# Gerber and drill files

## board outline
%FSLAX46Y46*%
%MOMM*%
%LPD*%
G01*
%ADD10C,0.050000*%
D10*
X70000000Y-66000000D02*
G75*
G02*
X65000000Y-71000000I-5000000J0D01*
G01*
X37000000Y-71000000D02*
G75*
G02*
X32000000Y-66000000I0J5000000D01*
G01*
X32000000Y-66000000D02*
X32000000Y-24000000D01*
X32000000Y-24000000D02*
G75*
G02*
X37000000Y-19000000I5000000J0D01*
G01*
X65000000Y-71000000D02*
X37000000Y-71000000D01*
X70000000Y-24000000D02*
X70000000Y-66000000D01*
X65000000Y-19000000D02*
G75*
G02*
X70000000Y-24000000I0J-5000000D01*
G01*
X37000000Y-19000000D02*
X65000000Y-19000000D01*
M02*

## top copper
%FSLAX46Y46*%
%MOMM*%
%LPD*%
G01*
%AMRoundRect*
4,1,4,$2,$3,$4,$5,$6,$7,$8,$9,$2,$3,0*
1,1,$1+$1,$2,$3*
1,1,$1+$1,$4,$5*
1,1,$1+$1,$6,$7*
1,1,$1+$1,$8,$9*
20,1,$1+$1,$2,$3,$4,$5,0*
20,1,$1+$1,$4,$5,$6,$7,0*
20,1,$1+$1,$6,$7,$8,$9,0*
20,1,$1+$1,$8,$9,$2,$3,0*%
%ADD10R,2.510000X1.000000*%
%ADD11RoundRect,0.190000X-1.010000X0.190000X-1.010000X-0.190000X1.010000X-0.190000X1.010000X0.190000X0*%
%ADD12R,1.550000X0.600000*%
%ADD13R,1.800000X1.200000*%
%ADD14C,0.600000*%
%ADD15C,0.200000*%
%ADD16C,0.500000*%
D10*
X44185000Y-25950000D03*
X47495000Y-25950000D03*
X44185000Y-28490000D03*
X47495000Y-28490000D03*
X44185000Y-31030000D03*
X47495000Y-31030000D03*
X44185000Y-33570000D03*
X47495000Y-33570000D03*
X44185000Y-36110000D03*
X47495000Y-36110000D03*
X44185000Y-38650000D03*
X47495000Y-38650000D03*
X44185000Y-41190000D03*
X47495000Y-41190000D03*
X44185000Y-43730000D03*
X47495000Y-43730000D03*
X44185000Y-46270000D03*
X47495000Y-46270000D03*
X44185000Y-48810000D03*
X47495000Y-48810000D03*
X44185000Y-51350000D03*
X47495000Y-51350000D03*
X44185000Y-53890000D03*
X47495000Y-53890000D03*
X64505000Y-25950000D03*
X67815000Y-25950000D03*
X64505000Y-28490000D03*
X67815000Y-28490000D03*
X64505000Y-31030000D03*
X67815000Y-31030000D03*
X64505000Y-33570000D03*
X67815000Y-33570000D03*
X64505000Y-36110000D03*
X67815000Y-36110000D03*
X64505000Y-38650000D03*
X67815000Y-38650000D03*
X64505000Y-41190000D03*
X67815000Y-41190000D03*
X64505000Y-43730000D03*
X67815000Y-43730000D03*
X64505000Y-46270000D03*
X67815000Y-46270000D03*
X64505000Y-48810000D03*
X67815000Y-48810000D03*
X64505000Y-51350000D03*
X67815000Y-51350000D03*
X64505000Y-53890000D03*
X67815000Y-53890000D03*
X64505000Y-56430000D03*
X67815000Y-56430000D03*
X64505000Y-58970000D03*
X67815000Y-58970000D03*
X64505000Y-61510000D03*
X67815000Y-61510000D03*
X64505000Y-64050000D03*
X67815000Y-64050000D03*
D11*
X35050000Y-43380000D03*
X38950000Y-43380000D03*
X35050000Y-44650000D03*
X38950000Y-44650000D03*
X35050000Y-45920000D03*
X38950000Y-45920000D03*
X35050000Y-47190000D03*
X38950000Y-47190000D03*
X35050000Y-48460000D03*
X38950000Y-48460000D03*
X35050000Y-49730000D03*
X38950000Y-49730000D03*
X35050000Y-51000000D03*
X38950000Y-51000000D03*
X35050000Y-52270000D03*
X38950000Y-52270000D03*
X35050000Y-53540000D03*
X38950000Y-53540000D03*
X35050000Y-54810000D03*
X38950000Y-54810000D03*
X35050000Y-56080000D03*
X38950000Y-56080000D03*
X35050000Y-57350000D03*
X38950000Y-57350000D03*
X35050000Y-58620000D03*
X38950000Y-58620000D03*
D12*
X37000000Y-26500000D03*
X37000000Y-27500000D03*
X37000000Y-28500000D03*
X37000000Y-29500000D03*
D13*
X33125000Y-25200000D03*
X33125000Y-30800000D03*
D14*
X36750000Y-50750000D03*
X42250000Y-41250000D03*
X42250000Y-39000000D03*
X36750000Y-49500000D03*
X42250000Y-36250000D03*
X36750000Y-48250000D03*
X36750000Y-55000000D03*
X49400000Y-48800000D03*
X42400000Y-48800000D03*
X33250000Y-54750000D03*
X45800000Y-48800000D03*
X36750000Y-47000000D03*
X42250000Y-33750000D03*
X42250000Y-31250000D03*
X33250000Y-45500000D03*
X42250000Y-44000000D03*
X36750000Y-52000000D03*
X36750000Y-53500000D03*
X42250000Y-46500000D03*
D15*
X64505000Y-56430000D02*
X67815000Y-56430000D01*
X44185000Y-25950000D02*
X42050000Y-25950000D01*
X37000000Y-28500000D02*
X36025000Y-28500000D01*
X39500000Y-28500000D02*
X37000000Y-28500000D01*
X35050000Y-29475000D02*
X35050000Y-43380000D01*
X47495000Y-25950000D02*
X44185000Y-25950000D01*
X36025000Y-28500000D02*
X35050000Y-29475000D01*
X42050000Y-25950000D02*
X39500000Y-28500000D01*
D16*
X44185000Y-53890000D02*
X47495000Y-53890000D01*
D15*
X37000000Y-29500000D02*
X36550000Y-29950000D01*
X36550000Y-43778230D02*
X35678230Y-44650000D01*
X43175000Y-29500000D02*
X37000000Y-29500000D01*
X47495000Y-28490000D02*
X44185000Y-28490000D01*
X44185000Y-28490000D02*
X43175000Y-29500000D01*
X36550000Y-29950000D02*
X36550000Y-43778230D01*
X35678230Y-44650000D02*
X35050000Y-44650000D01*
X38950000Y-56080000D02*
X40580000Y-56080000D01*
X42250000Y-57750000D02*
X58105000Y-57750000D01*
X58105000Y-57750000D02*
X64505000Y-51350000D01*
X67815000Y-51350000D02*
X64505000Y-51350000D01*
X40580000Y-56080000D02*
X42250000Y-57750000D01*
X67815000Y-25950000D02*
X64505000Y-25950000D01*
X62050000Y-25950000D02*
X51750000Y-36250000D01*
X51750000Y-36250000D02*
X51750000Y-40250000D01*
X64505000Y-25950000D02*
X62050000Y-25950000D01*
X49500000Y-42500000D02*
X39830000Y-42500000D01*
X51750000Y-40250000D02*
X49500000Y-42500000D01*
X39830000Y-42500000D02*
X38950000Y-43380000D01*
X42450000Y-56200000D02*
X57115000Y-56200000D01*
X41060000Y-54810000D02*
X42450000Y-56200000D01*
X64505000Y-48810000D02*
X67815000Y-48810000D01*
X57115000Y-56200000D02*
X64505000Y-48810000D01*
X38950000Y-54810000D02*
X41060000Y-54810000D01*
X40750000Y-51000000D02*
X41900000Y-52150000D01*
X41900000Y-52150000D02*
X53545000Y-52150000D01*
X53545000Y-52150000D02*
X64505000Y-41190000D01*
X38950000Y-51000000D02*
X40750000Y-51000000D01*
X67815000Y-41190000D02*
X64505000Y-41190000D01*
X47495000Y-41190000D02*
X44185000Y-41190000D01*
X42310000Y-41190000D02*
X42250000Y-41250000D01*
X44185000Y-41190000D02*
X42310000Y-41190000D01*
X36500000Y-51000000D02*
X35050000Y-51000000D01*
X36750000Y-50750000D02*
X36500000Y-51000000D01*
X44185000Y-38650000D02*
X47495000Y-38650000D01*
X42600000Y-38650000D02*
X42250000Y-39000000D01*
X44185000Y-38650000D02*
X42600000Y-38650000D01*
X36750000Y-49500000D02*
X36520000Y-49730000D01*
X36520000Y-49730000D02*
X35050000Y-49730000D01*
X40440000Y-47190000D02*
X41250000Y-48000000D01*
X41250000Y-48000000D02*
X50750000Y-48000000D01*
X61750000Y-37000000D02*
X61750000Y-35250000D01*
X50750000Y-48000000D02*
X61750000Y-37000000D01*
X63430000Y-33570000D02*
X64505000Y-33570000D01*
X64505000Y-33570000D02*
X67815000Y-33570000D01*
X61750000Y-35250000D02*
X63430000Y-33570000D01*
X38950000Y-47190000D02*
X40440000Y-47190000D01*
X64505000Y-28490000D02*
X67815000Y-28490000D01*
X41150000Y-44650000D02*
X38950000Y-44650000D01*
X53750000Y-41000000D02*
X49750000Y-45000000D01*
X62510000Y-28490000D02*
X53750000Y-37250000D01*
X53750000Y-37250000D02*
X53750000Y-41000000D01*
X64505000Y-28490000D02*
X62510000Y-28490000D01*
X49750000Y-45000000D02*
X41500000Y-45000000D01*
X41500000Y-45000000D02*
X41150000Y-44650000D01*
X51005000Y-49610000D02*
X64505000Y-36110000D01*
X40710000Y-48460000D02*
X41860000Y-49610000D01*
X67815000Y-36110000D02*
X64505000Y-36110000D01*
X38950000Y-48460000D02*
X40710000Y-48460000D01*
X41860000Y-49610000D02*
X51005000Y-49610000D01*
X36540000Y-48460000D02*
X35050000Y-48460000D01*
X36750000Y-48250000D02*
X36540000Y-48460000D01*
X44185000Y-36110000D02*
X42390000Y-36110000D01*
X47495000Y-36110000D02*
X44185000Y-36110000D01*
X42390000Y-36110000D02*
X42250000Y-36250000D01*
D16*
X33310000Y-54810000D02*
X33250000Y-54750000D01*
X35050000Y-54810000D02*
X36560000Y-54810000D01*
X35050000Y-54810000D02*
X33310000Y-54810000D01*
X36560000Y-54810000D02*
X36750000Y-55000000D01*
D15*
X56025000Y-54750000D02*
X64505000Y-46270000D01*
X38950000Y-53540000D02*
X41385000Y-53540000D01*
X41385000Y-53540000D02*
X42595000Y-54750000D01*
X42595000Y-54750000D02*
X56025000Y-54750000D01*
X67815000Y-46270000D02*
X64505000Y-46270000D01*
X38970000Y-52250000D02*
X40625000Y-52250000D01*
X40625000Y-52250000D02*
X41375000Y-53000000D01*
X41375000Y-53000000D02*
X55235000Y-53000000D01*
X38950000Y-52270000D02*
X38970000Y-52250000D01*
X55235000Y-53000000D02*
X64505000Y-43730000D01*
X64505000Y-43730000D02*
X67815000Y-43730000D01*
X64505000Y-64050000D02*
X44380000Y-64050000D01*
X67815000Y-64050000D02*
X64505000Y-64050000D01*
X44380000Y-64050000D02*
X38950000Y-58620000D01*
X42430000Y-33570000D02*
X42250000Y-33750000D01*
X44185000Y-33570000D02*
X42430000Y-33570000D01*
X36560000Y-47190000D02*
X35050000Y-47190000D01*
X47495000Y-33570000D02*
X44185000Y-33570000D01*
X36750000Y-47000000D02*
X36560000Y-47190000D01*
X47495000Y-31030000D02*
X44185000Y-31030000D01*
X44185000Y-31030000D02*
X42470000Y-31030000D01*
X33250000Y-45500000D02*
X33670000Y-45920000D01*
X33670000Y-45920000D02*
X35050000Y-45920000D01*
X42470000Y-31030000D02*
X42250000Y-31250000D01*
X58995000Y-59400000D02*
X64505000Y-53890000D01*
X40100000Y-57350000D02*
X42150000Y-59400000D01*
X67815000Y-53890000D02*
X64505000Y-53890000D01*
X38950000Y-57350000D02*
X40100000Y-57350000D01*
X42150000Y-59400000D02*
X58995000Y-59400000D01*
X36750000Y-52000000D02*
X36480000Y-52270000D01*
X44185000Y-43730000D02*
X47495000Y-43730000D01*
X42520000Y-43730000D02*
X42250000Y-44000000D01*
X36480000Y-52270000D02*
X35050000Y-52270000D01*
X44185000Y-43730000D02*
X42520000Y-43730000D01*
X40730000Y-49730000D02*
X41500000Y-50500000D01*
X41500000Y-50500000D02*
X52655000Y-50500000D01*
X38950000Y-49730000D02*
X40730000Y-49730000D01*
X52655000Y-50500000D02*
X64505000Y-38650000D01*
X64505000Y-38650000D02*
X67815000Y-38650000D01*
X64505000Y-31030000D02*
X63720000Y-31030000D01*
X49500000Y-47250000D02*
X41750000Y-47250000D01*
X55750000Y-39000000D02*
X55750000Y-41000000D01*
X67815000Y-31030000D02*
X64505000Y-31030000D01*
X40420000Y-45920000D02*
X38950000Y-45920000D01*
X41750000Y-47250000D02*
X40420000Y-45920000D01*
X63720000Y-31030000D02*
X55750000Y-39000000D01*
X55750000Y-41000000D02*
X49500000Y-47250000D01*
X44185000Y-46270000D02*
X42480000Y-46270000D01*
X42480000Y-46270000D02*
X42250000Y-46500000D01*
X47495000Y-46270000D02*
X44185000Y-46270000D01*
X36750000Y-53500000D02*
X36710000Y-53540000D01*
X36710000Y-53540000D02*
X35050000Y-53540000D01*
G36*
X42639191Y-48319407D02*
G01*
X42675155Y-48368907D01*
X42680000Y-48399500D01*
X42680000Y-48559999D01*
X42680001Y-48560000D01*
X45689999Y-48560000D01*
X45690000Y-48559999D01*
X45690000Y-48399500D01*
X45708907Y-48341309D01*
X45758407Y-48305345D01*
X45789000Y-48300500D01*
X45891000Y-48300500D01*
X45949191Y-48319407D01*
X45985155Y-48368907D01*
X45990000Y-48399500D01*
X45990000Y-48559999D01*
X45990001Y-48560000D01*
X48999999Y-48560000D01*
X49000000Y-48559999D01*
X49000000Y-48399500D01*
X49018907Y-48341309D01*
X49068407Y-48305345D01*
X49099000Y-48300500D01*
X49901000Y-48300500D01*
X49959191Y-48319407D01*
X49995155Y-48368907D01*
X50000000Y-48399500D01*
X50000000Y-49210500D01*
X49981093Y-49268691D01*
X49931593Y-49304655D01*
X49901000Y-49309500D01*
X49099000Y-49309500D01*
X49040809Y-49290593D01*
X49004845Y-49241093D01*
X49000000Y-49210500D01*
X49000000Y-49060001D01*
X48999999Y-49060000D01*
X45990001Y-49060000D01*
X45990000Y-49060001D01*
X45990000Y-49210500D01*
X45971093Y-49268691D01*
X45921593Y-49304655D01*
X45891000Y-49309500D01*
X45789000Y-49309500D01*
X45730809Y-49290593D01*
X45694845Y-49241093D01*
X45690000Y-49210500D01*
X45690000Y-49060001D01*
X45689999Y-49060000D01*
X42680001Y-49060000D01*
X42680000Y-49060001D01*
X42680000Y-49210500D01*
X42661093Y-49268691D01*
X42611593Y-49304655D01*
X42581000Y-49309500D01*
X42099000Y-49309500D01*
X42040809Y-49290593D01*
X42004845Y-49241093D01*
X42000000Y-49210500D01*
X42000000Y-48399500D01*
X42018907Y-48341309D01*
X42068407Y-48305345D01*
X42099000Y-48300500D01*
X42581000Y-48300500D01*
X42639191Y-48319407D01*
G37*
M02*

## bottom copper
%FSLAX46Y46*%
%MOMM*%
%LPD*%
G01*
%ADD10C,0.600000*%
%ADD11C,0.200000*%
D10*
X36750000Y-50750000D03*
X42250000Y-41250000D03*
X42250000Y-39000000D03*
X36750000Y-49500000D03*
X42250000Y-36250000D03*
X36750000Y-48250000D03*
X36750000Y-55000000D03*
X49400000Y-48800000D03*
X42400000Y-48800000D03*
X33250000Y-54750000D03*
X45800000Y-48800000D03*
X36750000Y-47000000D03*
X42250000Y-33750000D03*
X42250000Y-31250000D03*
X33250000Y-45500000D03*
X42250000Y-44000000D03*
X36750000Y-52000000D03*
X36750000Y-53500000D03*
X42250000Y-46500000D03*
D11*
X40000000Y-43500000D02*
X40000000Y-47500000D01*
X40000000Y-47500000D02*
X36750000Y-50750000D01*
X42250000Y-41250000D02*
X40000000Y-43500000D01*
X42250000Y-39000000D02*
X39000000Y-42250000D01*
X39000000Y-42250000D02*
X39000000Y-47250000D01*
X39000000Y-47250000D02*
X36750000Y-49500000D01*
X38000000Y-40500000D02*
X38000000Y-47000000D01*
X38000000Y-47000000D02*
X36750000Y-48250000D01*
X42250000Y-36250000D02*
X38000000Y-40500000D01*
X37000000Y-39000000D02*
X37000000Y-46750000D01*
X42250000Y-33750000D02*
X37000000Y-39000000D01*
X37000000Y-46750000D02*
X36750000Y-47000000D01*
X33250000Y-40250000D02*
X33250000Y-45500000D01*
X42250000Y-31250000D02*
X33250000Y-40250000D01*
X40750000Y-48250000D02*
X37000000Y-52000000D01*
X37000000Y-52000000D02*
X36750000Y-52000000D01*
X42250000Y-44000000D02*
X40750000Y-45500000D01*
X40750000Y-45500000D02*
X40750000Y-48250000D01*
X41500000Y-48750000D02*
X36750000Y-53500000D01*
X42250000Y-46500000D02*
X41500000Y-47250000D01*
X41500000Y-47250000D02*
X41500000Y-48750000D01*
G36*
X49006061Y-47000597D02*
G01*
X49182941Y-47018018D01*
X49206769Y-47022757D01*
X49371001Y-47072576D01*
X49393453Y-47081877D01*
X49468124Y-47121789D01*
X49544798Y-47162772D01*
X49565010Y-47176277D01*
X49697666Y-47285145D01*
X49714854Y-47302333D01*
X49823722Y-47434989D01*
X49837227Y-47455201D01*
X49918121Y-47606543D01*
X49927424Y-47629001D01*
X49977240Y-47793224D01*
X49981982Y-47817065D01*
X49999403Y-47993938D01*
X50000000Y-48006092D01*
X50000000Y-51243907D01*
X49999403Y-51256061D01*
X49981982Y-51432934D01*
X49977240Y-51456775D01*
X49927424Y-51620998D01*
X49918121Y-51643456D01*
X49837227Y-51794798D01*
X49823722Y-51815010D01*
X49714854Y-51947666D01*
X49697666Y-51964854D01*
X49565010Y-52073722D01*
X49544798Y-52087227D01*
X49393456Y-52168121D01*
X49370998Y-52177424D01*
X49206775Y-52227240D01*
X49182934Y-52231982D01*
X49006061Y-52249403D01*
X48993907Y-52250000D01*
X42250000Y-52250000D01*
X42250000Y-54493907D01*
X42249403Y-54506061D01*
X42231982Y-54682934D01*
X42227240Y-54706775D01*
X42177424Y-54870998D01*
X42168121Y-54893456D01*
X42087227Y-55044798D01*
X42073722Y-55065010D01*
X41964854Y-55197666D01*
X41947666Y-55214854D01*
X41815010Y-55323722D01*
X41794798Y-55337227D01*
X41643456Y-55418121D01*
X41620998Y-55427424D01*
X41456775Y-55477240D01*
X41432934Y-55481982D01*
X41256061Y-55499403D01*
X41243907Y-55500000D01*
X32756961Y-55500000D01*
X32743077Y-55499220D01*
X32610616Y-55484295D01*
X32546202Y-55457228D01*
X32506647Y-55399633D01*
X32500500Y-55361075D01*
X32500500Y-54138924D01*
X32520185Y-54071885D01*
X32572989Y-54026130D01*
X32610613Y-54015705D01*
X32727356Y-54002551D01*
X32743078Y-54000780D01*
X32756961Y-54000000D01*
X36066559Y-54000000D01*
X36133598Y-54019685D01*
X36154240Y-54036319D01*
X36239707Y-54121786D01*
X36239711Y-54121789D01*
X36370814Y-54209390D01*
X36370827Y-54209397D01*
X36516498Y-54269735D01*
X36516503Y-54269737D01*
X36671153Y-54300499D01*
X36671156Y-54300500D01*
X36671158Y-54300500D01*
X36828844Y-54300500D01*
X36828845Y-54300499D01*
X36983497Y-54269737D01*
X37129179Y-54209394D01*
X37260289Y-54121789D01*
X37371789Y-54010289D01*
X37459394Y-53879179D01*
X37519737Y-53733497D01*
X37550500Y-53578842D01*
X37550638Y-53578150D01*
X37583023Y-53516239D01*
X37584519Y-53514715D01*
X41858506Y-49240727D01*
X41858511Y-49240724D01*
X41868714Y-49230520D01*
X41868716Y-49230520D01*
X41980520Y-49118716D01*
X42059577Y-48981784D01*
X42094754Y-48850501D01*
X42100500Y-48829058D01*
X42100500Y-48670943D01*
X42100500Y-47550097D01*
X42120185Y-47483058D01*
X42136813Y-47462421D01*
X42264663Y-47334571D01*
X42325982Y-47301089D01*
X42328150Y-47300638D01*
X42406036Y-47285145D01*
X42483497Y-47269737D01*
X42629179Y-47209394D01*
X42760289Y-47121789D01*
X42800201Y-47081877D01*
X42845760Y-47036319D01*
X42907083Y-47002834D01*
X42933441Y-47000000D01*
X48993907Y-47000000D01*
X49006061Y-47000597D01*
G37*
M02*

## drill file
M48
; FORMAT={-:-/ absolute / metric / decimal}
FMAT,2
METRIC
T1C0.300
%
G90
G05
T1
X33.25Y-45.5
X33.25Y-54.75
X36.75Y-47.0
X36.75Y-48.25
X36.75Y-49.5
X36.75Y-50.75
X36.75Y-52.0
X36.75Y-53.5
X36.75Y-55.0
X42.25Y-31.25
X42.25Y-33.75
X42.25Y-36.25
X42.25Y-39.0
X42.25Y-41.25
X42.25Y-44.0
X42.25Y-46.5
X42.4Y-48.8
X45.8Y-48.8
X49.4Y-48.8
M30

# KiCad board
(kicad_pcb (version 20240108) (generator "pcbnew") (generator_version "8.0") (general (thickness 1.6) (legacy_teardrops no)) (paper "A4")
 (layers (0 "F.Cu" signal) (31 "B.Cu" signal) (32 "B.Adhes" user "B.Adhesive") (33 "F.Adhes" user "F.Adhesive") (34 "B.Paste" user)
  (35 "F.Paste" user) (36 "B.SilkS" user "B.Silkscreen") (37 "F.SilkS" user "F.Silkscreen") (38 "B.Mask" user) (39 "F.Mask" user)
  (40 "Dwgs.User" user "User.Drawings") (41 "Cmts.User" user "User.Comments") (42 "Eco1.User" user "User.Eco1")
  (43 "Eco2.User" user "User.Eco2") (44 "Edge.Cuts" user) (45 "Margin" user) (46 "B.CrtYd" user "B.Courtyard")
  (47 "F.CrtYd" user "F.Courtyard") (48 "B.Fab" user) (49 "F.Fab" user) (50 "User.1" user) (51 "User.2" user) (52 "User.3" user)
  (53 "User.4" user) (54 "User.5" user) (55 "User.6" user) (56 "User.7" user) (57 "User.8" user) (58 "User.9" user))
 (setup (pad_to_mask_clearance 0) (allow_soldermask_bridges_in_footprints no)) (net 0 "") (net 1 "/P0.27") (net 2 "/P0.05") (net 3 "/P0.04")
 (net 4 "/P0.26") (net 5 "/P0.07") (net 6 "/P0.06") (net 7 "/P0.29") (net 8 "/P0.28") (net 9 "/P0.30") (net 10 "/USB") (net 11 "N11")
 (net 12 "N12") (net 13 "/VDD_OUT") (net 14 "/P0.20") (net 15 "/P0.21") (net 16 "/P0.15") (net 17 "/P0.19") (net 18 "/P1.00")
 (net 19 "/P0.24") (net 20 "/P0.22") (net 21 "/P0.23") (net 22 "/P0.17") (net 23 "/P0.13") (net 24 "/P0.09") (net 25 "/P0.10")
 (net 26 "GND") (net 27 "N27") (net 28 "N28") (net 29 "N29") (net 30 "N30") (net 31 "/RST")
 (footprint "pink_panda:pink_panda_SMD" (layer "F.Cu") (at 56 45)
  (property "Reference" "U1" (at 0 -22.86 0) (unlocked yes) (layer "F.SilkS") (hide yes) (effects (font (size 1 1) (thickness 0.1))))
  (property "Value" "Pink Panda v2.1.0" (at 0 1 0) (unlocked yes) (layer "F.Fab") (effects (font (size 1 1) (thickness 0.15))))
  (pad "1" smd rect (at -11.815 -19.05) (size 2.51 1) (layers "F.Cu" "F.Paste" "F.Mask") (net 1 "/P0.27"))
  (pad "1" smd rect (at -8.505 -19.05) (size 2.51 1) (layers "F.Cu" "F.Paste" "F.Mask") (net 1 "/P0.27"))
  (pad "2" smd rect (at -11.815 -16.51) (size 2.51 1) (layers "F.Cu" "F.Paste" "F.Mask") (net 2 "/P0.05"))
  (pad "2" smd rect (at -8.505 -16.51) (size 2.51 1) (layers "F.Cu" "F.Paste" "F.Mask") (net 2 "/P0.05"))
  (pad "3" smd rect (at -11.815 -13.97) (size 2.51 1) (layers "F.Cu" "F.Paste" "F.Mask") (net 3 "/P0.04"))
  (pad "3" smd rect (at -8.505 -13.97) (size 2.51 1) (layers "F.Cu" "F.Paste" "F.Mask") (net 3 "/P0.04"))
  (pad "4" smd rect (at -11.815 -11.43) (size 2.51 1) (layers "F.Cu" "F.Paste" "F.Mask") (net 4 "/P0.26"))
  (pad "4" smd rect (at -8.505 -11.43) (size 2.51 1) (layers "F.Cu" "F.Paste" "F.Mask") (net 4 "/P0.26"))
  (pad "5" smd rect (at -11.815 -8.89) (size 2.51 1) (layers "F.Cu" "F.Paste" "F.Mask") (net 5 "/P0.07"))
  (pad "5" smd rect (at -8.505 -8.89) (size 2.51 1) (layers "F.Cu" "F.Paste" "F.Mask") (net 5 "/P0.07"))
  (pad "6" smd rect (at -11.815 -6.35) (size 2.51 1) (layers "F.Cu" "F.Paste" "F.Mask") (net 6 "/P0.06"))
  (pad "6" smd rect (at -8.505 -6.35) (size 2.51 1) (layers "F.Cu" "F.Paste" "F.Mask") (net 6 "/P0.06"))
  (pad "7" smd rect (at -11.815 -3.81) (size 2.51 1) (layers "F.Cu" "F.Paste" "F.Mask") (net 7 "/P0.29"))
  (pad "7" smd rect (at -8.505 -3.81) (size 2.51 1) (layers "F.Cu" "F.Paste" "F.Mask") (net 7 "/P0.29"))
  (pad "8" smd rect (at -11.815 -1.27) (size 2.51 1) (layers "F.Cu" "F.Paste" "F.Mask") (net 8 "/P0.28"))
  (pad "8" smd rect (at -8.505 -1.27) (size 2.51 1) (layers "F.Cu" "F.Paste" "F.Mask") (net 8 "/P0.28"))
  (pad "9" smd rect (at -11.815 1.27) (size 2.51 1) (layers "F.Cu" "F.Paste" "F.Mask") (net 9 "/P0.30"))
  (pad "9" smd rect (at -8.505 1.27) (size 2.51 1) (layers "F.Cu" "F.Paste" "F.Mask") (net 9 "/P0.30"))
  (pad "10" smd rect (at -11.815 3.81) (size 2.51 1) (layers "F.Cu" "F.Paste" "F.Mask") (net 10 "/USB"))
  (pad "10" smd rect (at -8.505 3.81) (size 2.51 1) (layers "F.Cu" "F.Paste" "F.Mask") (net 10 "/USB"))
  (pad "11" smd rect (at -11.815 6.35) (size 2.51 1) (layers "F.Cu" "F.Paste" "F.Mask") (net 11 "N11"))
  (pad "11" smd rect (at -8.505 6.35) (size 2.51 1) (layers "F.Cu" "F.Paste" "F.Mask") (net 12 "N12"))
  (pad "12" smd rect (at -11.815 8.89) (size 2.51 1) (layers "F.Cu" "F.Paste" "F.Mask") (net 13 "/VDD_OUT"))
  (pad "12" smd rect (at -8.505 8.89) (size 2.51 1) (layers "F.Cu" "F.Paste" "F.Mask") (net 13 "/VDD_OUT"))
  (pad "13" smd rect (at 8.505 -19.05) (size 2.51 1) (layers "F.Cu" "F.Paste" "F.Mask") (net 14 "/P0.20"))
  (pad "13" smd rect (at 11.815 -19.05) (size 2.51 1) (layers "F.Cu" "F.Paste" "F.Mask") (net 14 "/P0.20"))
  (pad "14" smd rect (at 8.505 -16.51) (size 2.51 1) (layers "F.Cu" "F.Paste" "F.Mask") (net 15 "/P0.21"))
  (pad "14" smd rect (at 11.815 -16.51) (size 2.51 1) (layers "F.Cu" "F.Paste" "F.Mask") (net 15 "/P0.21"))
  (pad "15" smd rect (at 8.505 -13.97) (size 2.51 1) (layers "F.Cu" "F.Paste" "F.Mask") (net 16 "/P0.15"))
  (pad "15" smd rect (at 11.815 -13.97) (size 2.51 1) (layers "F.Cu" "F.Paste" "F.Mask") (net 16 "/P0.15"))
  (pad "16" smd rect (at 8.505 -11.43) (size 2.51 1) (layers "F.Cu" "F.Paste" "F.Mask") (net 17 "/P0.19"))
  (pad "16" smd rect (at 11.815 -11.43) (size 2.51 1) (layers "F.Cu" "F.Paste" "F.Mask") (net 17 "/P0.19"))
  (pad "17" smd rect (at 8.505 -8.89) (size 2.51 1) (layers "F.Cu" "F.Paste" "F.Mask") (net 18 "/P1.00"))
  (pad "17" smd rect (at 11.815 -8.89) (size 2.51 1) (layers "F.Cu" "F.Paste" "F.Mask") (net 18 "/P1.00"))
  (pad "18" smd rect (at 8.505 -6.35) (size 2.51 1) (layers "F.Cu" "F.Paste" "F.Mask") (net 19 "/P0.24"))
  (pad "18" smd rect (at 11.815 -6.35) (size 2.51 1) (layers "F.Cu" "F.Paste" "F.Mask") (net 19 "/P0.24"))
  (pad "19" smd rect (at 8.505 -3.81) (size 2.51 1) (layers "F.Cu" "F.Paste" "F.Mask") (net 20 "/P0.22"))
  (pad "19" smd rect (at 11.815 -3.81) (size 2.51 1) (layers "F.Cu" "F.Paste" "F.Mask") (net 20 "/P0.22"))
  (pad "20" smd rect (at 8.505 -1.27) (size 2.51 1) (layers "F.Cu" "F.Paste" "F.Mask") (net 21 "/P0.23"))
  (pad "20" smd rect (at 11.815 -1.27) (size 2.51 1) (layers "F.Cu" "F.Paste" "F.Mask") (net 21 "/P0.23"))
  (pad "21" smd rect (at 8.505 1.27) (size 2.51 1) (layers "F.Cu" "F.Paste" "F.Mask") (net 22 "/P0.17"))
  (pad "21" smd rect (at 11.815 1.27) (size 2.51 1) (layers "F.Cu" "F.Paste" "F.Mask") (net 22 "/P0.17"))
  (pad "22" smd rect (at 8.505 3.81) (size 2.51 1) (layers "F.Cu" "F.Paste" "F.Mask") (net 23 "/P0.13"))
  (pad "22" smd rect (at 11.815 3.81) (size 2.51 1) (layers "F.Cu" "F.Paste" "F.Mask") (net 23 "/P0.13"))
  (pad "23" smd rect (at 8.505 6.35) (size 2.51 1) (layers "F.Cu" "F.Paste" "F.Mask") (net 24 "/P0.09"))
  (pad "23" smd rect (at 11.815 6.35) (size 2.51 1) (layers "F.Cu" "F.Paste" "F.Mask") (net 24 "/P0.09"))
  (pad "24" smd rect (at 8.505 8.89) (size 2.51 1) (layers "F.Cu" "F.Paste" "F.Mask") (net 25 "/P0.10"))
  (pad "24" smd rect (at 11.815 8.89) (size 2.51 1) (layers "F.Cu" "F.Paste" "F.Mask") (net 25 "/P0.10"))
  (pad "25" smd rect (at 8.505 11.43) (size 2.51 1) (layers "F.Cu" "F.Paste" "F.Mask") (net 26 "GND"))
  (pad "25" smd rect (at 11.815 11.43) (size 2.51 1) (layers "F.Cu" "F.Paste" "F.Mask") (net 26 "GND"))
  (pad "26" smd rect (at 8.505 13.97) (size 2.51 1) (layers "F.Cu" "F.Paste" "F.Mask") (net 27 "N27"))
  (pad "26" smd rect (at 11.815 13.97) (size 2.51 1) (layers "F.Cu" "F.Paste" "F.Mask") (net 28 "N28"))
  (pad "27" smd rect (at 8.505 16.51) (size 2.51 1) (layers "F.Cu" "F.Paste" "F.Mask") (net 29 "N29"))
  (pad "27" smd rect (at 11.815 16.51) (size 2.51 1) (layers "F.Cu" "F.Paste" "F.Mask") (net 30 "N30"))
  (pad "28" smd rect (at 8.505 19.05) (size 2.51 1) (layers "F.Cu" "F.Paste" "F.Mask") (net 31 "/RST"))
  (pad "28" smd rect (at 11.815 19.05) (size 2.51 1) (layers "F.Cu" "F.Paste" "F.Mask") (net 31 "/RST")))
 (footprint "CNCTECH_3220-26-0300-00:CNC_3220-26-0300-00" (layer "F.Cu") (at 37 51 -90)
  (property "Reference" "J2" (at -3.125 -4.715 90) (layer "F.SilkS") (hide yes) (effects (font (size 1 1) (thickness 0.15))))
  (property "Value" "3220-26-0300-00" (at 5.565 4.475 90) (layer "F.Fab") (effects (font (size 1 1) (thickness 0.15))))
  (pad "1" smd roundrect (at -7.62 1.95 270) (size 0.76 2.4) (layers "F.Cu" "F.Paste" "F.Mask") (roundrect_rratio 0.25) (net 1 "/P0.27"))
  (pad "2" smd roundrect (at -7.62 -1.95 270) (size 0.76 2.4) (layers "F.Cu" "F.Paste" "F.Mask") (roundrect_rratio 0.25) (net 14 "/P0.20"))
  (pad "3" smd roundrect (at -6.35 1.95 270) (size 0.76 2.4) (layers "F.Cu" "F.Paste" "F.Mask") (roundrect_rratio 0.25) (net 2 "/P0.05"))
  (pad "4" smd roundrect (at -6.35 -1.95 270) (size 0.76 2.4) (layers "F.Cu" "F.Paste" "F.Mask") (roundrect_rratio 0.25) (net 15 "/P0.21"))
  (pad "5" smd roundrect (at -5.08 1.95 270) (size 0.76 2.4) (layers "F.Cu" "F.Paste" "F.Mask") (roundrect_rratio 0.25) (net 3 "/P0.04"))
  (pad "6" smd roundrect (at -5.08 -1.95 270) (size 0.76 2.4) (layers "F.Cu" "F.Paste" "F.Mask") (roundrect_rratio 0.25) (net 16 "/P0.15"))
  (pad "7" smd roundrect (at -3.81 1.95 270) (size 0.76 2.4) (layers "F.Cu" "F.Paste" "F.Mask") (roundrect_rratio 0.25) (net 4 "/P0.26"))
  (pad "8" smd roundrect (at -3.81 -1.95 270) (size 0.76 2.4) (layers "F.Cu" "F.Paste" "F.Mask") (roundrect_rratio 0.25) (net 17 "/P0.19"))
  (pad "9" smd roundrect (at -2.54 1.95 270) (size 0.76 2.4) (layers "F.Cu" "F.Paste" "F.Mask") (roundrect_rratio 0.25) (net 5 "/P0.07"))
  (pad "10" smd roundrect (at -2.54 -1.95 270) (size 0.76 2.4) (layers "F.Cu" "F.Paste" "F.Mask") (roundrect_rratio 0.25) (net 18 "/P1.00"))
  (pad "11" smd roundrect (at -1.27 1.95 270) (size 0.76 2.4) (layers "F.Cu" "F.Paste" "F.Mask") (roundrect_rratio 0.25) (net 6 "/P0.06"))
  (pad "12" smd roundrect (at -1.27 -1.95 270) (size 0.76 2.4) (layers "F.Cu" "F.Paste" "F.Mask") (roundrect_rratio 0.25) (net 19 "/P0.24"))
  (pad "13" smd roundrect (at 0 1.95 270) (size 0.76 2.4) (layers "F.Cu" "F.Paste" "F.Mask") (roundrect_rratio 0.25) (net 7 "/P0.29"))
  (pad "14" smd roundrect (at 0 -1.95 270) (size 0.76 2.4) (layers "F.Cu" "F.Paste" "F.Mask") (roundrect_rratio 0.25) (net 20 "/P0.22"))
  (pad "15" smd roundrect (at 1.27 1.95 270) (size 0.76 2.4) (layers "F.Cu" "F.Paste" "F.Mask") (roundrect_rratio 0.25) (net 8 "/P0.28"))
  (pad "16" smd roundrect (at 1.27 -1.95 270) (size 0.76 2.4) (layers "F.Cu" "F.Paste" "F.Mask") (roundrect_rratio 0.25) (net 21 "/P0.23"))
  (pad "17" smd roundrect (at 2.54 1.95 270) (size 0.76 2.4) (layers "F.Cu" "F.Paste" "F.Mask") (roundrect_rratio 0.25) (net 9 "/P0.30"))
  (pad "18" smd roundrect (at 2.54 -1.95 270) (size 0.76 2.4) (layers "F.Cu" "F.Paste" "F.Mask") (roundrect_rratio 0.25) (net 22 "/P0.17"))
  (pad "19" smd roundrect (at 3.81 1.95 270) (size 0.76 2.4) (layers "F.Cu" "F.Paste" "F.Mask") (roundrect_rratio 0.25) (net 10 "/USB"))
  (pad "20" smd roundrect (at 3.81 -1.95 270) (size 0.76 2.4) (layers "F.Cu" "F.Paste" "F.Mask") (roundrect_rratio 0.25) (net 23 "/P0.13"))
  (pad "21" smd roundrect (at 5.08 1.95 270) (size 0.76 2.4) (layers "F.Cu" "F.Paste" "F.Mask") (roundrect_rratio 0.25) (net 13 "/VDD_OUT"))
  (pad "22" smd roundrect (at 5.08 -1.95 270) (size 0.76 2.4) (layers "F.Cu" "F.Paste" "F.Mask") (roundrect_rratio 0.25) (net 24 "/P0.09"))
  (pad "23" smd roundrect (at 6.35 1.95 270) (size 0.76 2.4) (layers "F.Cu" "F.Paste" "F.Mask") (roundrect_rratio 0.25) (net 26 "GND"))
  (pad "24" smd roundrect (at 6.35 -1.95 270) (size 0.76 2.4) (layers "F.Cu" "F.Paste" "F.Mask") (roundrect_rratio 0.25) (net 25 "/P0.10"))
  (pad "25" smd roundrect (at 7.62 1.95 270) (size 0.76 2.4) (layers "F.Cu" "F.Paste" "F.Mask") (roundrect_rratio 0.25) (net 26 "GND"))
  (pad "26" smd roundrect (at 7.62 -1.95 270) (size 0.76 2.4) (layers "F.Cu" "F.Paste" "F.Mask") (roundrect_rratio 0.25) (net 31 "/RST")))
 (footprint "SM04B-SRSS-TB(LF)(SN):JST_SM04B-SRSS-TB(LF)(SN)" (layer "F.Cu") (at 37 28 -90)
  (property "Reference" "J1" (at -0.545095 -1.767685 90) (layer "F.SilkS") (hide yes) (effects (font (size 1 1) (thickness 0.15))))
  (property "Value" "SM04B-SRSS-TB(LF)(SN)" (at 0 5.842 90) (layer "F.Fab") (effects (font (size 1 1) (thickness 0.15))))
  (pad "1" smd rect (at -1.5 0 270) (size 0.6 1.55) (layers "F.Cu" "F.Paste" "F.Mask") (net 26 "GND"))
  (pad "2" smd rect (at -0.5 0 270) (size 0.6 1.55) (layers "F.Cu" "F.Paste" "F.Mask") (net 13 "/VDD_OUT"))
  (pad "3" smd rect (at 0.5 0 270) (size 0.6 1.55) (layers "F.Cu" "F.Paste" "F.Mask") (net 1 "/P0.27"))
  (pad "4" smd rect (at 1.5 0 270) (size 0.6 1.55) (layers "F.Cu" "F.Paste" "F.Mask") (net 2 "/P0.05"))
  (pad "S1" smd rect (at -2.8 3.875 270) (size 1.2 1.8) (layers "F.Cu" "F.Paste" "F.Mask") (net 26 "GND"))
  (pad "S2" smd rect (at 2.8 3.875 270) (size 1.2 1.8) (layers "F.Cu" "F.Paste" "F.Mask") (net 26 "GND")))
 (gr_arc (start 70 66) (mid 68.535534 69.535534) (end 65 71) (stroke (width 0.05) (type default)) (layer "Edge.Cuts"))
 (gr_arc (start 37 71) (mid 33.464466 69.535534) (end 32 66) (stroke (width 0.05) (type default)) (layer "Edge.Cuts"))
 (gr_line (start 32 66) (end 32 24) (stroke (width 0.05) (type default)) (layer "Edge.Cuts"))
 (gr_arc (start 32 24) (mid 33.464466 20.464466) (end 37 19) (stroke (width 0.05) (type default)) (layer "Edge.Cuts"))
 (gr_line (start 65 71) (end 37 71) (stroke (width 0.05) (type default)) (layer "Edge.Cuts"))
 (gr_line (start 70 24) (end 70 66) (stroke (width 0.05) (type default)) (layer "Edge.Cuts"))
 (gr_arc (start 65 19) (mid 68.535534 20.464466) (end 70 24) (stroke (width 0.05) (type default)) (layer "Edge.Cuts"))
 (gr_line (start 37 19) (end 65 19) (stroke (width 0.05) (type default)) (layer "Edge.Cuts"))
 (segment (start 64.505 56.43) (end 67.815 56.43) (width 0.2) (layer "F.Cu") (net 26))
 (segment (start 44.185 25.95) (end 42.05 25.95) (width 0.2) (layer "F.Cu") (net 1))
 (segment (start 37 28.5) (end 36.025 28.5) (width 0.2) (layer "F.Cu") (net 1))
 (segment (start 39.5 28.5) (end 37 28.5) (width 0.2) (layer "F.Cu") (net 1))
 (segment (start 35.05 29.475) (end 35.05 43.38) (width 0.2) (layer "F.Cu") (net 1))
 (segment (start 47.495 25.95) (end 44.185 25.95) (width 0.2) (layer "F.Cu") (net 1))
 (segment (start 36.025 28.5) (end 35.05 29.475) (width 0.2) (layer "F.Cu") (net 1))
 (segment (start 42.05 25.95) (end 39.5 28.5) (width 0.2) (layer "F.Cu") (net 1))
 (segment (start 44.185 53.89) (end 47.495 53.89) (width 0.5) (layer "F.Cu") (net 13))
 (segment (start 37 29.5) (end 36.55 29.95) (width 0.2) (layer "F.Cu") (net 2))
 (segment (start 36.55 43.77823) (end 35.67823 44.65) (width 0.2) (layer "F.Cu") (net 2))
 (segment (start 43.175 29.5) (end 37 29.5) (width 0.2) (layer "F.Cu") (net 2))
 (segment (start 47.495 28.49) (end 44.185 28.49) (width 0.2) (layer "F.Cu") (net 2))
 (segment (start 44.185 28.49) (end 43.175 29.5) (width 0.2) (layer "F.Cu") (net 2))
 (segment (start 36.55 29.95) (end 36.55 43.77823) (width 0.2) (layer "F.Cu") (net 2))
 (segment (start 35.67823 44.65) (end 35.05 44.65) (width 0.2) (layer "F.Cu") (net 2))
 (segment (start 38.95 56.08) (end 40.58 56.08) (width 0.2) (layer "F.Cu") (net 24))
 (segment (start 42.25 57.75) (end 58.105 57.75) (width 0.2) (layer "F.Cu") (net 24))
 (segment (start 58.105 57.75) (end 64.505 51.35) (width 0.2) (layer "F.Cu") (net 24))
 (segment (start 67.815 51.35) (end 64.505 51.35) (width 0.2) (layer "F.Cu") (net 24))
 (segment (start 40.58 56.08) (end 42.25 57.75) (width 0.2) (layer "F.Cu") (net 24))
 (segment (start 67.815 25.95) (end 64.505 25.95) (width 0.2) (layer "F.Cu") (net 14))
 (segment (start 62.05 25.95) (end 51.75 36.25) (width 0.2) (layer "F.Cu") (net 14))
 (segment (start 51.75 36.25) (end 51.75 40.25) (width 0.2) (layer "F.Cu") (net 14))
 (segment (start 64.505 25.95) (end 62.05 25.95) (width 0.2) (layer "F.Cu") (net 14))
 (segment (start 49.5 42.5) (end 39.83 42.5) (width 0.2) (layer "F.Cu") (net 14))
 (segment (start 51.75 40.25) (end 49.5 42.5) (width 0.2) (layer "F.Cu") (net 14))
 (segment (start 39.83 42.5) (end 38.95 43.38) (width 0.2) (layer "F.Cu") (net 14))
 (segment (start 42.45 56.2) (end 57.115 56.2) (width 0.2) (layer "F.Cu") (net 23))
 (segment (start 41.06 54.81) (end 42.45 56.2) (width 0.2) (layer "F.Cu") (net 23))
 (segment (start 64.505 48.81) (end 67.815 48.81) (width 0.2) (layer "F.Cu") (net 23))
 (segment (start 57.115 56.2) (end 64.505 48.81) (width 0.2) (layer "F.Cu") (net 23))
 (segment (start 38.95 54.81) (end 41.06 54.81) (width 0.2) (layer "F.Cu") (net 23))
 (segment (start 40.75 51) (end 41.9 52.15) (width 0.2) (layer "F.Cu") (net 20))
 (segment (start 41.9 52.15) (end 53.545 52.15) (width 0.2) (layer "F.Cu") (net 20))
 (segment (start 53.545 52.15) (end 64.505 41.19) (width 0.2) (layer "F.Cu") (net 20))
 (segment (start 38.95 51) (end 40.75 51) (width 0.2) (layer "F.Cu") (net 20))
 (segment (start 67.815 41.19) (end 64.505 41.19) (width 0.2) (layer "F.Cu") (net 20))
 (segment (start 47.495 41.19) (end 44.185 41.19) (width 0.2) (layer "F.Cu") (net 7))
 (segment (start 42.31 41.19) (end 42.25 41.25) (width 0.2) (layer "F.Cu") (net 7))
 (segment (start 44.185 41.19) (end 42.31 41.19) (width 0.2) (layer "F.Cu") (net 7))
 (segment (start 36.5 51) (end 35.05 51) (width 0.2) (layer "F.Cu") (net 7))
 (segment (start 36.75 50.75) (end 36.5 51) (width 0.2) (layer "F.Cu") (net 7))
 (via (at 36.75 50.75) (size 0.6) (drill 0.3) (layers "F.Cu" "B.Cu") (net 7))
 (via (at 42.25 41.25) (size 0.6) (drill 0.3) (layers "F.Cu" "B.Cu") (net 7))
 (segment (start 40 43.5) (end 40 47.5) (width 0.2) (layer "B.Cu") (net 7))
 (segment (start 40 47.5) (end 36.75 50.75) (width 0.2) (layer "B.Cu") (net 7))
 (segment (start 42.25 41.25) (end 40 43.5) (width 0.2) (layer "B.Cu") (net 7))
 (segment (start 44.185 38.65) (end 47.495 38.65) (width 0.2) (layer "F.Cu") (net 6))
 (segment (start 42.6 38.65) (end 42.25 39) (width 0.2) (layer "F.Cu") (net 6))
 (segment (start 44.185 38.65) (end 42.6 38.65) (width 0.2) (layer "F.Cu") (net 6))
 (segment (start 36.75 49.5) (end 36.52 49.73) (width 0.2) (layer "F.Cu") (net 6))
 (segment (start 36.52 49.73) (end 35.05 49.73) (width 0.2) (layer "F.Cu") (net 6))
 (via (at 42.25 39) (size 0.6) (drill 0.3) (layers "F.Cu" "B.Cu") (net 6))
 (via (at 36.75 49.5) (size 0.6) (drill 0.3) (layers "F.Cu" "B.Cu") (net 6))
 (segment (start 42.25 39) (end 39 42.25) (width 0.2) (layer "B.Cu") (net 6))
 (segment (start 39 42.25) (end 39 47.25) (width 0.2) (layer "B.Cu") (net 6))
 (segment (start 39 47.25) (end 36.75 49.5) (width 0.2) (layer "B.Cu") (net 6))
 (segment (start 40.44 47.19) (end 41.25 48) (width 0.2) (layer "F.Cu") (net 17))
 (segment (start 41.25 48) (end 50.75 48) (width 0.2) (layer "F.Cu") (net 17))
 (segment (start 61.75 37) (end 61.75 35.25) (width 0.2) (layer "F.Cu") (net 17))
 (segment (start 50.75 48) (end 61.75 37) (width 0.2) (layer "F.Cu") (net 17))
 (segment (start 63.43 33.57) (end 64.505 33.57) (width 0.2) (layer "F.Cu") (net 17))
 (segment (start 64.505 33.57) (end 67.815 33.57) (width 0.2) (layer "F.Cu") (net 17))
 (segment (start 61.75 35.25) (end 63.43 33.57) (width 0.2) (layer "F.Cu") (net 17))
 (segment (start 38.95 47.19) (end 40.44 47.19) (width 0.2) (layer "F.Cu") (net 17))
 (segment (start 64.505 28.49) (end 67.815 28.49) (width 0.2) (layer "F.Cu") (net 15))
 (segment (start 41.15 44.65) (end 38.95 44.65) (width 0.2) (layer "F.Cu") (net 15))
 (segment (start 53.75 41) (end 49.75 45) (width 0.2) (layer "F.Cu") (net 15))
 (segment (start 62.51 28.49) (end 53.75 37.25) (width 0.2) (layer "F.Cu") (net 15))
 (segment (start 53.75 37.25) (end 53.75 41) (width 0.2) (layer "F.Cu") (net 15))
 (segment (start 64.505 28.49) (end 62.51 28.49) (width 0.2) (layer "F.Cu") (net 15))
 (segment (start 49.75 45) (end 41.5 45) (width 0.2) (layer "F.Cu") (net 15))
 (segment (start 41.5 45) (end 41.15 44.65) (width 0.2) (layer "F.Cu") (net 15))
 (segment (start 51.005 49.61) (end 64.505 36.11) (width 0.2) (layer "F.Cu") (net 18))
 (segment (start 40.71 48.46) (end 41.86 49.61) (width 0.2) (layer "F.Cu") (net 18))
 (segment (start 67.815 36.11) (end 64.505 36.11) (width 0.2) (layer "F.Cu") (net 18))
 (segment (start 38.95 48.46) (end 40.71 48.46) (width 0.2) (layer "F.Cu") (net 18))
 (segment (start 41.86 49.61) (end 51.005 49.61) (width 0.2) (layer "F.Cu") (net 18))
 (segment (start 36.54 48.46) (end 35.05 48.46) (width 0.2) (layer "F.Cu") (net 5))
 (segment (start 36.75 48.25) (end 36.54 48.46) (width 0.2) (layer "F.Cu") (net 5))
 (segment (start 44.185 36.11) (end 42.39 36.11) (width 0.2) (layer "F.Cu") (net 5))
 (segment (start 47.495 36.11) (end 44.185 36.11) (width 0.2) (layer "F.Cu") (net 5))
 (segment (start 42.39 36.11) (end 42.25 36.25) (width 0.2) (layer "F.Cu") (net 5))
 (via (at 42.25 36.25) (size 0.6) (drill 0.3) (layers "F.Cu" "B.Cu") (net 5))
 (via (at 36.75 48.25) (size 0.6) (drill 0.3) (layers "F.Cu" "B.Cu") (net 5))
 (segment (start 38 40.5) (end 38 47) (width 0.2) (layer "B.Cu") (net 5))
 (segment (start 38 47) (end 36.75 48.25) (width 0.2) (layer "B.Cu") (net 5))
 (segment (start 42.25 36.25) (end 38 40.5) (width 0.2) (layer "B.Cu") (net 5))
 (segment (start 33.31 54.81) (end 33.25 54.75) (width 0.5) (layer "F.Cu") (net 10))
 (segment (start 35.05 54.81) (end 36.56 54.81) (width 0.5) (layer "F.Cu") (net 10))
 (segment (start 35.05 54.81) (end 33.31 54.81) (width 0.5) (layer "F.Cu") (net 10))
 (segment (start 36.56 54.81) (end 36.75 55) (width 0.5) (layer "F.Cu") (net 10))
 (via (at 36.75 55) (size 0.6) (drill 0.3) (layers "F.Cu" "B.Cu") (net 10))
 (via (at 49.4 48.8) (size 0.6) (drill 0.3) (layers "F.Cu" "B.Cu") (free yes) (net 10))
 (via (at 42.4 48.8) (size 0.6) (drill 0.3) (layers "F.Cu" "B.Cu") (free yes) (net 10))
 (via (at 33.25 54.75) (size 0.6) (drill 0.3) (layers "F.Cu" "B.Cu") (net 10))
 (via (at 45.8 48.8) (size 0.6) (drill 0.3) (layers "F.Cu" "B.Cu") (free yes) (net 10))
 (segment (start 56.025 54.75) (end 64.505 46.27) (width 0.2) (layer "F.Cu") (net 22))
 (segment (start 38.95 53.54) (end 41.385 53.54) (width 0.2) (layer "F.Cu") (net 22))
 (segment (start 41.385 53.54) (end 42.595 54.75) (width 0.2) (layer "F.Cu") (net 22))
 (segment (start 42.595 54.75) (end 56.025 54.75) (width 0.2) (layer "F.Cu") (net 22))
 (segment (start 67.815 46.27) (end 64.505 46.27) (width 0.2) (layer "F.Cu") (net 22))
 (segment (start 38.97 52.25) (end 40.625 52.25) (width 0.2) (layer "F.Cu") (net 21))
 (segment (start 40.625 52.25) (end 41.375 53) (width 0.2) (layer "F.Cu") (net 21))
 (segment (start 41.375 53) (end 55.235 53) (width 0.2) (layer "F.Cu") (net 21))
 (segment (start 38.95 52.27) (end 38.97 52.25) (width 0.2) (layer "F.Cu") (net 21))
 (segment (start 55.235 53) (end 64.505 43.73) (width 0.2) (layer "F.Cu") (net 21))
 (segment (start 64.505 43.73) (end 67.815 43.73) (width 0.2) (layer "F.Cu") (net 21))
 (segment (start 64.505 64.05) (end 44.38 64.05) (width 0.2) (layer "F.Cu") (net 31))
 (segment (start 67.815 64.05) (end 64.505 64.05) (width 0.2) (layer "F.Cu") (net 31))
 (segment (start 44.38 64.05) (end 38.95 58.62) (width 0.2) (layer "F.Cu") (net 31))
 (segment (start 42.43 33.57) (end 42.25 33.75) (width 0.2) (layer "F.Cu") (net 4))
 (segment (start 44.185 33.57) (end 42.43 33.57) (width 0.2) (layer "F.Cu") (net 4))
 (segment (start 36.56 47.19) (end 35.05 47.19) (width 0.2) (layer "F.Cu") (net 4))
 (segment (start 47.495 33.57) (end 44.185 33.57) (width 0.2) (layer "F.Cu") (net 4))
 (segment (start 36.75 47) (end 36.56 47.19) (width 0.2) (layer "F.Cu") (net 4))
 (via (at 36.75 47) (size 0.6) (drill 0.3) (layers "F.Cu" "B.Cu") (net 4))
 (via (at 42.25 33.75) (size 0.6) (drill 0.3) (layers "F.Cu" "B.Cu") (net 4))
 (segment (start 37 39) (end 37 46.75) (width 0.2) (layer "B.Cu") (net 4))
 (segment (start 42.25 33.75) (end 37 39) (width 0.2) (layer "B.Cu") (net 4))
 (segment (start 37 46.75) (end 36.75 47) (width 0.2) (layer "B.Cu") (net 4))
 (segment (start 47.495 31.03) (end 44.185 31.03) (width 0.2) (layer "F.Cu") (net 3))
 (segment (start 44.185 31.03) (end 42.47 31.03) (width 0.2) (layer "F.Cu") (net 3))
 (segment (start 33.25 45.5) (end 33.67 45.92) (width 0.2) (layer "F.Cu") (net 3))
 (segment (start 33.67 45.92) (end 35.05 45.92) (width 0.2) (layer "F.Cu") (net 3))
 (segment (start 42.47 31.03) (end 42.25 31.25) (width 0.2) (layer "F.Cu") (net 3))
 (via (at 42.25 31.25) (size 0.6) (drill 0.3) (layers "F.Cu" "B.Cu") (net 3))
 (via (at 33.25 45.5) (size 0.6) (drill 0.3) (layers "F.Cu" "B.Cu") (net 3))
 (segment (start 33.25 40.25) (end 33.25 45.5) (width 0.2) (layer "B.Cu") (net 3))
 (segment (start 42.25 31.25) (end 33.25 40.25) (width 0.2) (layer "B.Cu") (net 3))
 (segment (start 58.995 59.4) (end 64.505 53.89) (width 0.2) (layer "F.Cu") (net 25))
 (segment (start 40.1 57.35) (end 42.15 59.4) (width 0.2) (layer "F.Cu") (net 25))
 (segment (start 67.815 53.89) (end 64.505 53.89) (width 0.2) (layer "F.Cu") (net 25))
 (segment (start 38.95 57.35) (end 40.1 57.35) (width 0.2) (layer "F.Cu") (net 25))
 (segment (start 42.15 59.4) (end 58.995 59.4) (width 0.2) (layer "F.Cu") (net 25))
 (segment (start 36.75 52) (end 36.48 52.27) (width 0.2) (layer "F.Cu") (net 8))
 (segment (start 44.185 43.73) (end 47.495 43.73) (width 0.2) (layer "F.Cu") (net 8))
 (segment (start 42.52 43.73) (end 42.25 44) (width 0.2) (layer "F.Cu") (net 8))
 (segment (start 36.48 52.27) (end 35.05 52.27) (width 0.2) (layer "F.Cu") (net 8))
 (segment (start 44.185 43.73) (end 42.52 43.73) (width 0.2) (layer "F.Cu") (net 8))
 (via (at 42.25 44) (size 0.6) (drill 0.3) (layers "F.Cu" "B.Cu") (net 8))
 (via (at 36.75 52) (size 0.6) (drill 0.3) (layers "F.Cu" "B.Cu") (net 8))
 (segment (start 40.75 48.25) (end 37 52) (width 0.2) (layer "B.Cu") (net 8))
 (segment (start 37 52) (end 36.75 52) (width 0.2) (layer "B.Cu") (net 8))
 (segment (start 42.25 44) (end 40.75 45.5) (width 0.2) (layer "B.Cu") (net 8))
 (segment (start 40.75 45.5) (end 40.75 48.25) (width 0.2) (layer "B.Cu") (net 8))
 (segment (start 40.73 49.73) (end 41.5 50.5) (width 0.2) (layer "F.Cu") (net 19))
 (segment (start 41.5 50.5) (end 52.655 50.5) (width 0.2) (layer "F.Cu") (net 19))
 (segment (start 38.95 49.73) (end 40.73 49.73) (width 0.2) (layer "F.Cu") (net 19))
 (segment (start 52.655 50.5) (end 64.505 38.65) (width 0.2) (layer "F.Cu") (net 19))
 (segment (start 64.505 38.65) (end 67.815 38.65) (width 0.2) (layer "F.Cu") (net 19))
 (segment (start 64.505 31.03) (end 63.72 31.03) (width 0.2) (layer "F.Cu") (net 16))
 (segment (start 49.5 47.25) (end 41.75 47.25) (width 0.2) (layer "F.Cu") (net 16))
 (segment (start 55.75 39) (end 55.75 41) (width 0.2) (layer "F.Cu") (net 16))
 (segment (start 67.815 31.03) (end 64.505 31.03) (width 0.2) (layer "F.Cu") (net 16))
 (segment (start 40.42 45.92) (end 38.95 45.92) (width 0.2) (layer "F.Cu") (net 16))
 (segment (start 41.75 47.25) (end 40.42 45.92) (width 0.2) (layer "F.Cu") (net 16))
 (segment (start 63.72 31.03) (end 55.75 39) (width 0.2) (layer "F.Cu") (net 16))
 (segment (start 55.75 41) (end 49.5 47.25) (width 0.2) (layer "F.Cu") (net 16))
 (segment (start 44.185 46.27) (end 42.48 46.27) (width 0.2) (layer "F.Cu") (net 9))
 (segment (start 42.48 46.27) (end 42.25 46.5) (width 0.2) (layer "F.Cu") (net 9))
 (segment (start 47.495 46.27) (end 44.185 46.27) (width 0.2) (layer "F.Cu") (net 9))
 (segment (start 36.75 53.5) (end 36.71 53.54) (width 0.2) (layer "F.Cu") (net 9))
 (segment (start 36.71 53.54) (end 35.05 53.54) (width 0.2) (layer "F.Cu") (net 9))
 (via (at 36.75 53.5) (size 0.6) (drill 0.3) (layers "F.Cu" "B.Cu") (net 9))
 (via (at 42.25 46.5) (size 0.6) (drill 0.3) (layers "F.Cu" "B.Cu") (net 9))
 (segment (start 41.5 48.75) (end 36.75 53.5) (width 0.2) (layer "B.Cu") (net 9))
 (segment (start 42.25 46.5) (end 41.5 47.25) (width 0.2) (layer "B.Cu") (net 9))
 (segment (start 41.5 47.25) (end 41.5 48.75) (width 0.2) (layer "B.Cu") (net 9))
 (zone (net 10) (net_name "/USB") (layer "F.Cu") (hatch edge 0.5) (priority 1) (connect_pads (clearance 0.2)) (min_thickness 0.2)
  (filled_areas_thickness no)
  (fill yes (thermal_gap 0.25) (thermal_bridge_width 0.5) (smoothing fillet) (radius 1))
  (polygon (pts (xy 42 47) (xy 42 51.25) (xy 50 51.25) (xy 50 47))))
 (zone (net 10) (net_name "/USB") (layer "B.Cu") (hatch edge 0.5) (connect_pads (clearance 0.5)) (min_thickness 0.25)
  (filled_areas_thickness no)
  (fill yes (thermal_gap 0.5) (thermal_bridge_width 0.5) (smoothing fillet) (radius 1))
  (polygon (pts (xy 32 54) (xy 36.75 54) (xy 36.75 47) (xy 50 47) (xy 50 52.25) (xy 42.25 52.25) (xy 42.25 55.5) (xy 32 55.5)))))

